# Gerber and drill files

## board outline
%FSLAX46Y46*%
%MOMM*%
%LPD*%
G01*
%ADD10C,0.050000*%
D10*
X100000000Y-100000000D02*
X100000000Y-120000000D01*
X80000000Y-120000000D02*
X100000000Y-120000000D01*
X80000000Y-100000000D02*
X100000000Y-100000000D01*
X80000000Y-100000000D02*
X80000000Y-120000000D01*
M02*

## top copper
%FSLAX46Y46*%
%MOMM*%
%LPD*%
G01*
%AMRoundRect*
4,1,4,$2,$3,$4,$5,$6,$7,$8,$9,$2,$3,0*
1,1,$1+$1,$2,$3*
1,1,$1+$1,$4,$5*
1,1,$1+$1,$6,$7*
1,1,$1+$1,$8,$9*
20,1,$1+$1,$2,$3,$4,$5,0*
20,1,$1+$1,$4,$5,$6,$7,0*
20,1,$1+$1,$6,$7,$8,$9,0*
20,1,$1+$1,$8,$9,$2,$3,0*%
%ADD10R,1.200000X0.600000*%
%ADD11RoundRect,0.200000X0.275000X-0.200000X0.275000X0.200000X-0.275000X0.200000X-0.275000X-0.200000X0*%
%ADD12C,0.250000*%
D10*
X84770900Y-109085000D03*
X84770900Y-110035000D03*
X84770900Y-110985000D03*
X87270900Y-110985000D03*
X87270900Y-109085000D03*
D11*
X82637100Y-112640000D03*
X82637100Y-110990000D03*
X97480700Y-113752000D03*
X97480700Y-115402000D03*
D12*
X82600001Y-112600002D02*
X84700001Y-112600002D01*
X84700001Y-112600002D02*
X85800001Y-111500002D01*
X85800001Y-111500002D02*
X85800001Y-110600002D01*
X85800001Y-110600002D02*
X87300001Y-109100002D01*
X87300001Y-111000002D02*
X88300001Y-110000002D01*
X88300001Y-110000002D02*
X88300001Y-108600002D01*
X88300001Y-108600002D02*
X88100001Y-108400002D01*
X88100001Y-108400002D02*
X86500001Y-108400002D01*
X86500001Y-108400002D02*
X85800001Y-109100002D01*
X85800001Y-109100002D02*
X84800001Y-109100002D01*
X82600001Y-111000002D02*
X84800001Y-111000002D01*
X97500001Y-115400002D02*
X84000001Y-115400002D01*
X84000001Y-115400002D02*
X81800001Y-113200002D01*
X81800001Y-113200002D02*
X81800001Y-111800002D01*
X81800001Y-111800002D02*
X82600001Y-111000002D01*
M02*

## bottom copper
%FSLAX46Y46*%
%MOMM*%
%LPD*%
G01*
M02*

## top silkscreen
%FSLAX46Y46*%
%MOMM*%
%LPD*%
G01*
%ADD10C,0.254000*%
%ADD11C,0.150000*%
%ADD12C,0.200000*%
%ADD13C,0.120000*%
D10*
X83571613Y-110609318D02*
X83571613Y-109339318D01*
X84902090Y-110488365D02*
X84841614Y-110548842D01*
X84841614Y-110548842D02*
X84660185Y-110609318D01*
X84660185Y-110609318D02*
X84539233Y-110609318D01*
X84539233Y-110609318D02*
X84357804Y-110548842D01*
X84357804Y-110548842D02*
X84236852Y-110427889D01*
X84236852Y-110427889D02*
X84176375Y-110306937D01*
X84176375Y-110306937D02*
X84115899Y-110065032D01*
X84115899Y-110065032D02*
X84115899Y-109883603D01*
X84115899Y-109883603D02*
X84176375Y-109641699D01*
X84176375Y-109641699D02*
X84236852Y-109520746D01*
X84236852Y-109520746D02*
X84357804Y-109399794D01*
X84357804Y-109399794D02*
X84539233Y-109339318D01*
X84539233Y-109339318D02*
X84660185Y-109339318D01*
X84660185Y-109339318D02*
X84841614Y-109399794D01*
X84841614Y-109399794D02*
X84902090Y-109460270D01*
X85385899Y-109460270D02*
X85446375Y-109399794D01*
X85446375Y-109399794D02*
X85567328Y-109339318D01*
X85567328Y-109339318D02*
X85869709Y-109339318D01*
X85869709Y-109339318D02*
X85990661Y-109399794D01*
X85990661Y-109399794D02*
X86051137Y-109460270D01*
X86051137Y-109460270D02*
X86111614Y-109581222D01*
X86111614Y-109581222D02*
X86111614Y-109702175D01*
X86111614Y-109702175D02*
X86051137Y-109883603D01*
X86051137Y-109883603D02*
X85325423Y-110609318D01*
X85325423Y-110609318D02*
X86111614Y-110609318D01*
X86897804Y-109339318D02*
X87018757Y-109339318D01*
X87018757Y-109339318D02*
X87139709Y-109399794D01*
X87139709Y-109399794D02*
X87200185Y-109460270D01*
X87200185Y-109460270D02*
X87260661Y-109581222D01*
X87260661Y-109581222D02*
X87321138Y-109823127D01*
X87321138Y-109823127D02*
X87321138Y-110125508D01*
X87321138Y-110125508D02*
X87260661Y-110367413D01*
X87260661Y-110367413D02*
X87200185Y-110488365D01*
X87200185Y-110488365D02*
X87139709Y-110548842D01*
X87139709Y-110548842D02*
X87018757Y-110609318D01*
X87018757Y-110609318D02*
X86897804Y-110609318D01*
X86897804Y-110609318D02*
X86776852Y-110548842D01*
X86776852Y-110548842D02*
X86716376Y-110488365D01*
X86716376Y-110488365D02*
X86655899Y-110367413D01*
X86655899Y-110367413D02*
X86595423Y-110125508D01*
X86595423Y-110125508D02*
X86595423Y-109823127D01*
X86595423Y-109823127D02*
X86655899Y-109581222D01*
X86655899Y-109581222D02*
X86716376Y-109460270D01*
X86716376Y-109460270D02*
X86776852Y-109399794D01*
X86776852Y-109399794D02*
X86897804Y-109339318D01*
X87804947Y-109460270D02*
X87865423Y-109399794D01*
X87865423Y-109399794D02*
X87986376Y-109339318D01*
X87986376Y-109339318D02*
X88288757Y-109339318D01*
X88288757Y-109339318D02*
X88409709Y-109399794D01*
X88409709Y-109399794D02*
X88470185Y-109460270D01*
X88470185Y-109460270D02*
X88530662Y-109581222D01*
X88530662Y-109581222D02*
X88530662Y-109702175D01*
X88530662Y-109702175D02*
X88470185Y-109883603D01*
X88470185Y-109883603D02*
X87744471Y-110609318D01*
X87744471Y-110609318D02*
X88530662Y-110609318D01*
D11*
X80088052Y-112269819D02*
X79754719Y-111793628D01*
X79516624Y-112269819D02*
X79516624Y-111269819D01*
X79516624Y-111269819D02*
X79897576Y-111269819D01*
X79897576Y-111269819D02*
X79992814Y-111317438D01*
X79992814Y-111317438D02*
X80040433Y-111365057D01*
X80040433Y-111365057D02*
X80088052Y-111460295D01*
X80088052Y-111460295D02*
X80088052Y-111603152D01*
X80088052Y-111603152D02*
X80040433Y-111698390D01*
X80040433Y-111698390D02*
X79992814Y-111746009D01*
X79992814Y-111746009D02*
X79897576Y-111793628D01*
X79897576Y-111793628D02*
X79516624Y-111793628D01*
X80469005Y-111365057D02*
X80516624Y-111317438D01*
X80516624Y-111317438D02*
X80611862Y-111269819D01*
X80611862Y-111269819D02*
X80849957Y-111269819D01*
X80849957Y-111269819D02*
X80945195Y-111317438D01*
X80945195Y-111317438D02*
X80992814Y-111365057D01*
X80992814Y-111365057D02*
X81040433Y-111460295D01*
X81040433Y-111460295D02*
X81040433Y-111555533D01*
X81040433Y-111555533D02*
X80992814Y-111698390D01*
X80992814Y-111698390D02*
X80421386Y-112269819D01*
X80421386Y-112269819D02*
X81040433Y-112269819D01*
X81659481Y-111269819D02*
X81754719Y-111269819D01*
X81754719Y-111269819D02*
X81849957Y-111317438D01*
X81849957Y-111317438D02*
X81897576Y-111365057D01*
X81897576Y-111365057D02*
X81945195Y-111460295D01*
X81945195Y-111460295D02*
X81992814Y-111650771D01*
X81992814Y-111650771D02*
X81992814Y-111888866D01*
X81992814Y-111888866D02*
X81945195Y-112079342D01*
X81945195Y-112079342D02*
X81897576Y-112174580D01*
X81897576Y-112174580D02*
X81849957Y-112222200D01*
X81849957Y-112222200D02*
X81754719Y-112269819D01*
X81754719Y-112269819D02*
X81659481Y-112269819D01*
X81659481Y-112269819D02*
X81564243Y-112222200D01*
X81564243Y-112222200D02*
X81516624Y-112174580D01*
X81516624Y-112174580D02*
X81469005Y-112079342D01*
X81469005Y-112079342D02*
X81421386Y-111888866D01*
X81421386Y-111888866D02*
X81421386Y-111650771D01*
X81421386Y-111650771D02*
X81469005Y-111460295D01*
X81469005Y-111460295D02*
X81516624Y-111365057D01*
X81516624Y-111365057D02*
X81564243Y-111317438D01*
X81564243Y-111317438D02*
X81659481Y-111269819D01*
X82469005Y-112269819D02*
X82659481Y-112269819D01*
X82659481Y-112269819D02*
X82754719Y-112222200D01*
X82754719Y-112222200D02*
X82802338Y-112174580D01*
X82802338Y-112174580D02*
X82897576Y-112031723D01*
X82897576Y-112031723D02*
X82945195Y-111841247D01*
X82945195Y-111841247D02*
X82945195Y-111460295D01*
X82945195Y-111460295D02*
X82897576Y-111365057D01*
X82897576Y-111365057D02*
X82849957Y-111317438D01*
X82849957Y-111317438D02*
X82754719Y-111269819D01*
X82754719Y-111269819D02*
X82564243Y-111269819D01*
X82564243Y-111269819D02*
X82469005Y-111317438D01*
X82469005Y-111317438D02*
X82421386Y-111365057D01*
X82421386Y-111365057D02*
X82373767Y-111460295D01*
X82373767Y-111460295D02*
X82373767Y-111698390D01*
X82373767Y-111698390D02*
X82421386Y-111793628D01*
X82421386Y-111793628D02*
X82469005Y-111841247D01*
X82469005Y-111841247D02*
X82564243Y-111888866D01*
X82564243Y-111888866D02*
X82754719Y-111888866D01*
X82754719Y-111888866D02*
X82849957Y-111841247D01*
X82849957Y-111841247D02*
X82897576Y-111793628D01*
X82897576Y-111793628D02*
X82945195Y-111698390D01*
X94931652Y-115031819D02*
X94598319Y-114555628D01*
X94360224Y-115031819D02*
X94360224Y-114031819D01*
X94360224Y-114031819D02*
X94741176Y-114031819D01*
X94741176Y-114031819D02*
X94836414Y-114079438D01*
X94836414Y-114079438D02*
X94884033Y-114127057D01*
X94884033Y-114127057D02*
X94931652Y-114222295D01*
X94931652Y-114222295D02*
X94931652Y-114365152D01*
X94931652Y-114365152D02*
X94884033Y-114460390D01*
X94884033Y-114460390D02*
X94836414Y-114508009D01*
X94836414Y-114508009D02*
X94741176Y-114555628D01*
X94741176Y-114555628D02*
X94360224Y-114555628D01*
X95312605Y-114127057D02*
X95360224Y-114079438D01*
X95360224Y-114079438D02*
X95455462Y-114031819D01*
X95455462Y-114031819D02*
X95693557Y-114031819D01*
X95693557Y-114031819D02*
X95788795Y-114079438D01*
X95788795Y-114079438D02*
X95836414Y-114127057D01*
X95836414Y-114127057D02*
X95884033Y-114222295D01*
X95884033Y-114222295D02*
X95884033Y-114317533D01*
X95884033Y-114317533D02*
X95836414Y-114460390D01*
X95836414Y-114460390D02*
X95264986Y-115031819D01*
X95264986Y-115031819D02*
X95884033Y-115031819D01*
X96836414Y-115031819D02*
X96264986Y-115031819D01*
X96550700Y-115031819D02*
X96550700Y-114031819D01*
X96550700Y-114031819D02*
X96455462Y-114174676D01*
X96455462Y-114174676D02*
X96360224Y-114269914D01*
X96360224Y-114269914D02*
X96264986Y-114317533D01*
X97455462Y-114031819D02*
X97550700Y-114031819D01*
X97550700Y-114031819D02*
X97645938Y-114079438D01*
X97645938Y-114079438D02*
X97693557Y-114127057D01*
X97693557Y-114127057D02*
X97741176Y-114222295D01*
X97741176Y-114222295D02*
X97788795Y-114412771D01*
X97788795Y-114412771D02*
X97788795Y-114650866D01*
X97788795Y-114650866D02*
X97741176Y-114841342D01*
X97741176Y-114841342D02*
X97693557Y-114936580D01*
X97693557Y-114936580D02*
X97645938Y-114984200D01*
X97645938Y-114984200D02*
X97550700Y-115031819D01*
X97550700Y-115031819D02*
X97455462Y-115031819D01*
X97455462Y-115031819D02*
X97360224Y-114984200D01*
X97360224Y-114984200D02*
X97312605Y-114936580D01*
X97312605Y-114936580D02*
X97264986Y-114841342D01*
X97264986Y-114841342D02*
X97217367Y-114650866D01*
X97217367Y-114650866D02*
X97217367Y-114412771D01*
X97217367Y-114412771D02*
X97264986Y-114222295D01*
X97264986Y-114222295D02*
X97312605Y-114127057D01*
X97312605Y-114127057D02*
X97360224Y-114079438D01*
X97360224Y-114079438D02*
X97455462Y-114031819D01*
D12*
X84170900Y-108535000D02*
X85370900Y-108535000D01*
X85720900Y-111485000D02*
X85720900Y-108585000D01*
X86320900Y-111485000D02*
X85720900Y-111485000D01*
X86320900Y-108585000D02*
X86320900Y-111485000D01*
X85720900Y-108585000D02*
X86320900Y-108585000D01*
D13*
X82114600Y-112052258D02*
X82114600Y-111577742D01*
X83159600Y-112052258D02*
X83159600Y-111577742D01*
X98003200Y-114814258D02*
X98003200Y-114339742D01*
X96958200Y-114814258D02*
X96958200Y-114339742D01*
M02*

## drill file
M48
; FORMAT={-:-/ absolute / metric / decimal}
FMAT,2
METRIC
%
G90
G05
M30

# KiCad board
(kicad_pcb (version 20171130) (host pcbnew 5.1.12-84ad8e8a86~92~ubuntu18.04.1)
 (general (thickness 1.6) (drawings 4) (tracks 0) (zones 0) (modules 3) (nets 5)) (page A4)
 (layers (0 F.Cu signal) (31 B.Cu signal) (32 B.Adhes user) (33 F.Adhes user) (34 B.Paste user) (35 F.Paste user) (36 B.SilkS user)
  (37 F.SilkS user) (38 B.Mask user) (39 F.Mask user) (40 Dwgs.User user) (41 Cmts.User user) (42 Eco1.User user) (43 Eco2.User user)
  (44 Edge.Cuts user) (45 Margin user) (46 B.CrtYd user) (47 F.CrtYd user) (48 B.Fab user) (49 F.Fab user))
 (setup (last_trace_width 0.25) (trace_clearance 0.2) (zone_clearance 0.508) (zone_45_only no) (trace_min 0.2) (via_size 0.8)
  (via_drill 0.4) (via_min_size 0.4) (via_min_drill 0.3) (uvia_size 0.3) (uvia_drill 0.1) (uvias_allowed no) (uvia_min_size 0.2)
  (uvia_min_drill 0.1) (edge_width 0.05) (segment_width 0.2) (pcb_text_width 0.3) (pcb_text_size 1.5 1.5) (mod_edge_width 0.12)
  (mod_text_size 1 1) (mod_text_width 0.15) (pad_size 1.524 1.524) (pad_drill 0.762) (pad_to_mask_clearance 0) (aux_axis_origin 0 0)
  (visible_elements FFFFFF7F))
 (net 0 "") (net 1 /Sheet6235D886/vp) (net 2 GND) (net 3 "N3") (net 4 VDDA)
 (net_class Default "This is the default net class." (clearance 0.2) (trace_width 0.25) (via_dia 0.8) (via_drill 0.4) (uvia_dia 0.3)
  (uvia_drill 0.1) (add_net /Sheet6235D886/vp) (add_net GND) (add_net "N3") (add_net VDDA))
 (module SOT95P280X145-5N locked (layer F.Cu) (at 86.020900 110.035000)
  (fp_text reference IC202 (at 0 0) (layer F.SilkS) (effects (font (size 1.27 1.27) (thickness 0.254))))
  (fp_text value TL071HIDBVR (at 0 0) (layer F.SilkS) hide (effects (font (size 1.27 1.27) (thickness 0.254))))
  (fp_line (start -1.85 -1.5) (end -0.65 -1.5) (layer F.SilkS) (width 0.2))
  (fp_line (start -0.3 1.45) (end -0.3 -1.45) (layer F.SilkS) (width 0.2))
  (fp_line (start 0.3 1.45) (end -0.3 1.45) (layer F.SilkS) (width 0.2))
  (fp_line (start 0.3 -1.45) (end 0.3 1.45) (layer F.SilkS) (width 0.2))
  (fp_line (start -0.3 -1.45) (end 0.3 -1.45) (layer F.SilkS) (width 0.2))
  (pad 1 smd rect (at -1.25 -0.95 90.000000) (size 0.6 1.2) (layers F.Cu F.Mask F.Paste) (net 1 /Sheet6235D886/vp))
  (pad 2 smd rect (at -1.25 0 90.000000) (size 0.6 1.2) (layers F.Cu F.Mask F.Paste) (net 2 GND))
  (pad 3 smd rect (at -1.25 0.95 90.000000) (size 0.6 1.2) (layers F.Cu F.Mask F.Paste) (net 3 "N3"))
  (pad 4 smd rect (at 1.25 0.95 90.000000) (size 0.6 1.2) (layers F.Cu F.Mask F.Paste) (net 1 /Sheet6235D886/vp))
  (pad 5 smd rect (at 1.25 -0.95 90.000000) (size 0.6 1.2) (layers F.Cu F.Mask F.Paste) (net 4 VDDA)))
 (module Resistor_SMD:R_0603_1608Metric (layer F.Cu) (at 82.637100 111.815000 90.000000)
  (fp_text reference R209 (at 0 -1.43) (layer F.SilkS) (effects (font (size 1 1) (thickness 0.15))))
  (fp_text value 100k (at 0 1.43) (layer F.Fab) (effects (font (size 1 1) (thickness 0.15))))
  (fp_line (start -0.237258 -0.5225) (end 0.237258 -0.5225) (layer F.SilkS) (width 0.12))
  (fp_line (start -0.237258 0.5225) (end 0.237258 0.5225) (layer F.SilkS) (width 0.12))
  (pad 1 smd roundrect (at -0.825 0 90.000000) (size 0.8 0.95) (layers F.Cu F.Mask F.Paste) (roundrect_rratio 0.25) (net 4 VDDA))
  (pad 2 smd roundrect (at 0.825 0 90.000000) (size 0.8 0.95) (layers F.Cu F.Mask F.Paste) (roundrect_rratio 0.25) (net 3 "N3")))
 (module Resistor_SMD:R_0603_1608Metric (layer F.Cu) (at 97.480700 114.577000 90.000000)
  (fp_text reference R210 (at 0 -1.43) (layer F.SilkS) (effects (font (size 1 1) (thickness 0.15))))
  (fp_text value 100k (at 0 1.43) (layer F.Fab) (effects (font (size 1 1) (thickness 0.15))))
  (fp_line (start -0.237258 0.5225) (end 0.237258 0.5225) (layer F.SilkS) (width 0.12))
  (fp_line (start -0.237258 -0.5225) (end 0.237258 -0.5225) (layer F.SilkS) (width 0.12))
  (pad 2 smd roundrect (at 0.825 0 90.000000) (size 0.8 0.95) (layers F.Cu F.Mask F.Paste) (roundrect_rratio 0.25) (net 2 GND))
  (pad 1 smd roundrect (at -0.825 0 90.000000) (size 0.8 0.95) (layers F.Cu F.Mask F.Paste) (roundrect_rratio 0.25) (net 3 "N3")))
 (gr_line (start 100 100) (end 100 120) (layer Edge.Cuts) (width 0.05))
 (gr_line (start 80 120) (end 100 120) (layer Edge.Cuts) (width 0.05))
 (gr_line (start 80 100) (end 100 100) (layer Edge.Cuts) (width 0.05))
 (gr_line (start 80 100) (end 80 120) (layer Edge.Cuts) (width 0.05))
 (segment (start 82.600001 112.600002) (end 84.700001 112.600002) (width 0.250000) (layer F.Cu) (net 4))
 (segment (start 84.700001 112.600002) (end 85.800001 111.500002) (width 0.250000) (layer F.Cu) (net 4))
 (segment (start 85.800001 111.500002) (end 85.800001 110.600002) (width 0.250000) (layer F.Cu) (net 4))
 (segment (start 85.800001 110.600002) (end 87.300001 109.100002) (width 0.250000) (layer F.Cu) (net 4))
 (segment (start 87.300001 111.000002) (end 88.300001 110.000002) (width 0.250000) (layer F.Cu) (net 1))
 (segment (start 88.300001 110.000002) (end 88.300001 108.600002) (width 0.250000) (layer F.Cu) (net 1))
 (segment (start 88.300001 108.600002) (end 88.100001 108.400002) (width 0.250000) (layer F.Cu) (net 1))
 (segment (start 88.100001 108.400002) (end 86.500001 108.400002) (width 0.250000) (layer F.Cu) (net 1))
 (segment (start 86.500001 108.400002) (end 85.800001 109.100002) (width 0.250000) (layer F.Cu) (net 1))
 (segment (start 85.800001 109.100002) (end 84.800001 109.100002) (width 0.250000) (layer F.Cu) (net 1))
 (segment (start 82.600001 111.000002) (end 84.800001 111.000002) (width 0.250000) (layer F.Cu) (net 3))
 (segment (start 97.500001 115.400002) (end 84.000001 115.400002) (width 0.250000) (layer F.Cu) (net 3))
 (segment (start 84.000001 115.400002) (end 81.800001 113.200002) (width 0.250000) (layer F.Cu) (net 3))
 (segment (start 81.800001 113.200002) (end 81.800001 111.800002) (width 0.250000) (layer F.Cu) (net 3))
 (segment (start 81.800001 111.800002) (end 82.600001 111.000002) (width 0.250000) (layer F.Cu) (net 3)))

